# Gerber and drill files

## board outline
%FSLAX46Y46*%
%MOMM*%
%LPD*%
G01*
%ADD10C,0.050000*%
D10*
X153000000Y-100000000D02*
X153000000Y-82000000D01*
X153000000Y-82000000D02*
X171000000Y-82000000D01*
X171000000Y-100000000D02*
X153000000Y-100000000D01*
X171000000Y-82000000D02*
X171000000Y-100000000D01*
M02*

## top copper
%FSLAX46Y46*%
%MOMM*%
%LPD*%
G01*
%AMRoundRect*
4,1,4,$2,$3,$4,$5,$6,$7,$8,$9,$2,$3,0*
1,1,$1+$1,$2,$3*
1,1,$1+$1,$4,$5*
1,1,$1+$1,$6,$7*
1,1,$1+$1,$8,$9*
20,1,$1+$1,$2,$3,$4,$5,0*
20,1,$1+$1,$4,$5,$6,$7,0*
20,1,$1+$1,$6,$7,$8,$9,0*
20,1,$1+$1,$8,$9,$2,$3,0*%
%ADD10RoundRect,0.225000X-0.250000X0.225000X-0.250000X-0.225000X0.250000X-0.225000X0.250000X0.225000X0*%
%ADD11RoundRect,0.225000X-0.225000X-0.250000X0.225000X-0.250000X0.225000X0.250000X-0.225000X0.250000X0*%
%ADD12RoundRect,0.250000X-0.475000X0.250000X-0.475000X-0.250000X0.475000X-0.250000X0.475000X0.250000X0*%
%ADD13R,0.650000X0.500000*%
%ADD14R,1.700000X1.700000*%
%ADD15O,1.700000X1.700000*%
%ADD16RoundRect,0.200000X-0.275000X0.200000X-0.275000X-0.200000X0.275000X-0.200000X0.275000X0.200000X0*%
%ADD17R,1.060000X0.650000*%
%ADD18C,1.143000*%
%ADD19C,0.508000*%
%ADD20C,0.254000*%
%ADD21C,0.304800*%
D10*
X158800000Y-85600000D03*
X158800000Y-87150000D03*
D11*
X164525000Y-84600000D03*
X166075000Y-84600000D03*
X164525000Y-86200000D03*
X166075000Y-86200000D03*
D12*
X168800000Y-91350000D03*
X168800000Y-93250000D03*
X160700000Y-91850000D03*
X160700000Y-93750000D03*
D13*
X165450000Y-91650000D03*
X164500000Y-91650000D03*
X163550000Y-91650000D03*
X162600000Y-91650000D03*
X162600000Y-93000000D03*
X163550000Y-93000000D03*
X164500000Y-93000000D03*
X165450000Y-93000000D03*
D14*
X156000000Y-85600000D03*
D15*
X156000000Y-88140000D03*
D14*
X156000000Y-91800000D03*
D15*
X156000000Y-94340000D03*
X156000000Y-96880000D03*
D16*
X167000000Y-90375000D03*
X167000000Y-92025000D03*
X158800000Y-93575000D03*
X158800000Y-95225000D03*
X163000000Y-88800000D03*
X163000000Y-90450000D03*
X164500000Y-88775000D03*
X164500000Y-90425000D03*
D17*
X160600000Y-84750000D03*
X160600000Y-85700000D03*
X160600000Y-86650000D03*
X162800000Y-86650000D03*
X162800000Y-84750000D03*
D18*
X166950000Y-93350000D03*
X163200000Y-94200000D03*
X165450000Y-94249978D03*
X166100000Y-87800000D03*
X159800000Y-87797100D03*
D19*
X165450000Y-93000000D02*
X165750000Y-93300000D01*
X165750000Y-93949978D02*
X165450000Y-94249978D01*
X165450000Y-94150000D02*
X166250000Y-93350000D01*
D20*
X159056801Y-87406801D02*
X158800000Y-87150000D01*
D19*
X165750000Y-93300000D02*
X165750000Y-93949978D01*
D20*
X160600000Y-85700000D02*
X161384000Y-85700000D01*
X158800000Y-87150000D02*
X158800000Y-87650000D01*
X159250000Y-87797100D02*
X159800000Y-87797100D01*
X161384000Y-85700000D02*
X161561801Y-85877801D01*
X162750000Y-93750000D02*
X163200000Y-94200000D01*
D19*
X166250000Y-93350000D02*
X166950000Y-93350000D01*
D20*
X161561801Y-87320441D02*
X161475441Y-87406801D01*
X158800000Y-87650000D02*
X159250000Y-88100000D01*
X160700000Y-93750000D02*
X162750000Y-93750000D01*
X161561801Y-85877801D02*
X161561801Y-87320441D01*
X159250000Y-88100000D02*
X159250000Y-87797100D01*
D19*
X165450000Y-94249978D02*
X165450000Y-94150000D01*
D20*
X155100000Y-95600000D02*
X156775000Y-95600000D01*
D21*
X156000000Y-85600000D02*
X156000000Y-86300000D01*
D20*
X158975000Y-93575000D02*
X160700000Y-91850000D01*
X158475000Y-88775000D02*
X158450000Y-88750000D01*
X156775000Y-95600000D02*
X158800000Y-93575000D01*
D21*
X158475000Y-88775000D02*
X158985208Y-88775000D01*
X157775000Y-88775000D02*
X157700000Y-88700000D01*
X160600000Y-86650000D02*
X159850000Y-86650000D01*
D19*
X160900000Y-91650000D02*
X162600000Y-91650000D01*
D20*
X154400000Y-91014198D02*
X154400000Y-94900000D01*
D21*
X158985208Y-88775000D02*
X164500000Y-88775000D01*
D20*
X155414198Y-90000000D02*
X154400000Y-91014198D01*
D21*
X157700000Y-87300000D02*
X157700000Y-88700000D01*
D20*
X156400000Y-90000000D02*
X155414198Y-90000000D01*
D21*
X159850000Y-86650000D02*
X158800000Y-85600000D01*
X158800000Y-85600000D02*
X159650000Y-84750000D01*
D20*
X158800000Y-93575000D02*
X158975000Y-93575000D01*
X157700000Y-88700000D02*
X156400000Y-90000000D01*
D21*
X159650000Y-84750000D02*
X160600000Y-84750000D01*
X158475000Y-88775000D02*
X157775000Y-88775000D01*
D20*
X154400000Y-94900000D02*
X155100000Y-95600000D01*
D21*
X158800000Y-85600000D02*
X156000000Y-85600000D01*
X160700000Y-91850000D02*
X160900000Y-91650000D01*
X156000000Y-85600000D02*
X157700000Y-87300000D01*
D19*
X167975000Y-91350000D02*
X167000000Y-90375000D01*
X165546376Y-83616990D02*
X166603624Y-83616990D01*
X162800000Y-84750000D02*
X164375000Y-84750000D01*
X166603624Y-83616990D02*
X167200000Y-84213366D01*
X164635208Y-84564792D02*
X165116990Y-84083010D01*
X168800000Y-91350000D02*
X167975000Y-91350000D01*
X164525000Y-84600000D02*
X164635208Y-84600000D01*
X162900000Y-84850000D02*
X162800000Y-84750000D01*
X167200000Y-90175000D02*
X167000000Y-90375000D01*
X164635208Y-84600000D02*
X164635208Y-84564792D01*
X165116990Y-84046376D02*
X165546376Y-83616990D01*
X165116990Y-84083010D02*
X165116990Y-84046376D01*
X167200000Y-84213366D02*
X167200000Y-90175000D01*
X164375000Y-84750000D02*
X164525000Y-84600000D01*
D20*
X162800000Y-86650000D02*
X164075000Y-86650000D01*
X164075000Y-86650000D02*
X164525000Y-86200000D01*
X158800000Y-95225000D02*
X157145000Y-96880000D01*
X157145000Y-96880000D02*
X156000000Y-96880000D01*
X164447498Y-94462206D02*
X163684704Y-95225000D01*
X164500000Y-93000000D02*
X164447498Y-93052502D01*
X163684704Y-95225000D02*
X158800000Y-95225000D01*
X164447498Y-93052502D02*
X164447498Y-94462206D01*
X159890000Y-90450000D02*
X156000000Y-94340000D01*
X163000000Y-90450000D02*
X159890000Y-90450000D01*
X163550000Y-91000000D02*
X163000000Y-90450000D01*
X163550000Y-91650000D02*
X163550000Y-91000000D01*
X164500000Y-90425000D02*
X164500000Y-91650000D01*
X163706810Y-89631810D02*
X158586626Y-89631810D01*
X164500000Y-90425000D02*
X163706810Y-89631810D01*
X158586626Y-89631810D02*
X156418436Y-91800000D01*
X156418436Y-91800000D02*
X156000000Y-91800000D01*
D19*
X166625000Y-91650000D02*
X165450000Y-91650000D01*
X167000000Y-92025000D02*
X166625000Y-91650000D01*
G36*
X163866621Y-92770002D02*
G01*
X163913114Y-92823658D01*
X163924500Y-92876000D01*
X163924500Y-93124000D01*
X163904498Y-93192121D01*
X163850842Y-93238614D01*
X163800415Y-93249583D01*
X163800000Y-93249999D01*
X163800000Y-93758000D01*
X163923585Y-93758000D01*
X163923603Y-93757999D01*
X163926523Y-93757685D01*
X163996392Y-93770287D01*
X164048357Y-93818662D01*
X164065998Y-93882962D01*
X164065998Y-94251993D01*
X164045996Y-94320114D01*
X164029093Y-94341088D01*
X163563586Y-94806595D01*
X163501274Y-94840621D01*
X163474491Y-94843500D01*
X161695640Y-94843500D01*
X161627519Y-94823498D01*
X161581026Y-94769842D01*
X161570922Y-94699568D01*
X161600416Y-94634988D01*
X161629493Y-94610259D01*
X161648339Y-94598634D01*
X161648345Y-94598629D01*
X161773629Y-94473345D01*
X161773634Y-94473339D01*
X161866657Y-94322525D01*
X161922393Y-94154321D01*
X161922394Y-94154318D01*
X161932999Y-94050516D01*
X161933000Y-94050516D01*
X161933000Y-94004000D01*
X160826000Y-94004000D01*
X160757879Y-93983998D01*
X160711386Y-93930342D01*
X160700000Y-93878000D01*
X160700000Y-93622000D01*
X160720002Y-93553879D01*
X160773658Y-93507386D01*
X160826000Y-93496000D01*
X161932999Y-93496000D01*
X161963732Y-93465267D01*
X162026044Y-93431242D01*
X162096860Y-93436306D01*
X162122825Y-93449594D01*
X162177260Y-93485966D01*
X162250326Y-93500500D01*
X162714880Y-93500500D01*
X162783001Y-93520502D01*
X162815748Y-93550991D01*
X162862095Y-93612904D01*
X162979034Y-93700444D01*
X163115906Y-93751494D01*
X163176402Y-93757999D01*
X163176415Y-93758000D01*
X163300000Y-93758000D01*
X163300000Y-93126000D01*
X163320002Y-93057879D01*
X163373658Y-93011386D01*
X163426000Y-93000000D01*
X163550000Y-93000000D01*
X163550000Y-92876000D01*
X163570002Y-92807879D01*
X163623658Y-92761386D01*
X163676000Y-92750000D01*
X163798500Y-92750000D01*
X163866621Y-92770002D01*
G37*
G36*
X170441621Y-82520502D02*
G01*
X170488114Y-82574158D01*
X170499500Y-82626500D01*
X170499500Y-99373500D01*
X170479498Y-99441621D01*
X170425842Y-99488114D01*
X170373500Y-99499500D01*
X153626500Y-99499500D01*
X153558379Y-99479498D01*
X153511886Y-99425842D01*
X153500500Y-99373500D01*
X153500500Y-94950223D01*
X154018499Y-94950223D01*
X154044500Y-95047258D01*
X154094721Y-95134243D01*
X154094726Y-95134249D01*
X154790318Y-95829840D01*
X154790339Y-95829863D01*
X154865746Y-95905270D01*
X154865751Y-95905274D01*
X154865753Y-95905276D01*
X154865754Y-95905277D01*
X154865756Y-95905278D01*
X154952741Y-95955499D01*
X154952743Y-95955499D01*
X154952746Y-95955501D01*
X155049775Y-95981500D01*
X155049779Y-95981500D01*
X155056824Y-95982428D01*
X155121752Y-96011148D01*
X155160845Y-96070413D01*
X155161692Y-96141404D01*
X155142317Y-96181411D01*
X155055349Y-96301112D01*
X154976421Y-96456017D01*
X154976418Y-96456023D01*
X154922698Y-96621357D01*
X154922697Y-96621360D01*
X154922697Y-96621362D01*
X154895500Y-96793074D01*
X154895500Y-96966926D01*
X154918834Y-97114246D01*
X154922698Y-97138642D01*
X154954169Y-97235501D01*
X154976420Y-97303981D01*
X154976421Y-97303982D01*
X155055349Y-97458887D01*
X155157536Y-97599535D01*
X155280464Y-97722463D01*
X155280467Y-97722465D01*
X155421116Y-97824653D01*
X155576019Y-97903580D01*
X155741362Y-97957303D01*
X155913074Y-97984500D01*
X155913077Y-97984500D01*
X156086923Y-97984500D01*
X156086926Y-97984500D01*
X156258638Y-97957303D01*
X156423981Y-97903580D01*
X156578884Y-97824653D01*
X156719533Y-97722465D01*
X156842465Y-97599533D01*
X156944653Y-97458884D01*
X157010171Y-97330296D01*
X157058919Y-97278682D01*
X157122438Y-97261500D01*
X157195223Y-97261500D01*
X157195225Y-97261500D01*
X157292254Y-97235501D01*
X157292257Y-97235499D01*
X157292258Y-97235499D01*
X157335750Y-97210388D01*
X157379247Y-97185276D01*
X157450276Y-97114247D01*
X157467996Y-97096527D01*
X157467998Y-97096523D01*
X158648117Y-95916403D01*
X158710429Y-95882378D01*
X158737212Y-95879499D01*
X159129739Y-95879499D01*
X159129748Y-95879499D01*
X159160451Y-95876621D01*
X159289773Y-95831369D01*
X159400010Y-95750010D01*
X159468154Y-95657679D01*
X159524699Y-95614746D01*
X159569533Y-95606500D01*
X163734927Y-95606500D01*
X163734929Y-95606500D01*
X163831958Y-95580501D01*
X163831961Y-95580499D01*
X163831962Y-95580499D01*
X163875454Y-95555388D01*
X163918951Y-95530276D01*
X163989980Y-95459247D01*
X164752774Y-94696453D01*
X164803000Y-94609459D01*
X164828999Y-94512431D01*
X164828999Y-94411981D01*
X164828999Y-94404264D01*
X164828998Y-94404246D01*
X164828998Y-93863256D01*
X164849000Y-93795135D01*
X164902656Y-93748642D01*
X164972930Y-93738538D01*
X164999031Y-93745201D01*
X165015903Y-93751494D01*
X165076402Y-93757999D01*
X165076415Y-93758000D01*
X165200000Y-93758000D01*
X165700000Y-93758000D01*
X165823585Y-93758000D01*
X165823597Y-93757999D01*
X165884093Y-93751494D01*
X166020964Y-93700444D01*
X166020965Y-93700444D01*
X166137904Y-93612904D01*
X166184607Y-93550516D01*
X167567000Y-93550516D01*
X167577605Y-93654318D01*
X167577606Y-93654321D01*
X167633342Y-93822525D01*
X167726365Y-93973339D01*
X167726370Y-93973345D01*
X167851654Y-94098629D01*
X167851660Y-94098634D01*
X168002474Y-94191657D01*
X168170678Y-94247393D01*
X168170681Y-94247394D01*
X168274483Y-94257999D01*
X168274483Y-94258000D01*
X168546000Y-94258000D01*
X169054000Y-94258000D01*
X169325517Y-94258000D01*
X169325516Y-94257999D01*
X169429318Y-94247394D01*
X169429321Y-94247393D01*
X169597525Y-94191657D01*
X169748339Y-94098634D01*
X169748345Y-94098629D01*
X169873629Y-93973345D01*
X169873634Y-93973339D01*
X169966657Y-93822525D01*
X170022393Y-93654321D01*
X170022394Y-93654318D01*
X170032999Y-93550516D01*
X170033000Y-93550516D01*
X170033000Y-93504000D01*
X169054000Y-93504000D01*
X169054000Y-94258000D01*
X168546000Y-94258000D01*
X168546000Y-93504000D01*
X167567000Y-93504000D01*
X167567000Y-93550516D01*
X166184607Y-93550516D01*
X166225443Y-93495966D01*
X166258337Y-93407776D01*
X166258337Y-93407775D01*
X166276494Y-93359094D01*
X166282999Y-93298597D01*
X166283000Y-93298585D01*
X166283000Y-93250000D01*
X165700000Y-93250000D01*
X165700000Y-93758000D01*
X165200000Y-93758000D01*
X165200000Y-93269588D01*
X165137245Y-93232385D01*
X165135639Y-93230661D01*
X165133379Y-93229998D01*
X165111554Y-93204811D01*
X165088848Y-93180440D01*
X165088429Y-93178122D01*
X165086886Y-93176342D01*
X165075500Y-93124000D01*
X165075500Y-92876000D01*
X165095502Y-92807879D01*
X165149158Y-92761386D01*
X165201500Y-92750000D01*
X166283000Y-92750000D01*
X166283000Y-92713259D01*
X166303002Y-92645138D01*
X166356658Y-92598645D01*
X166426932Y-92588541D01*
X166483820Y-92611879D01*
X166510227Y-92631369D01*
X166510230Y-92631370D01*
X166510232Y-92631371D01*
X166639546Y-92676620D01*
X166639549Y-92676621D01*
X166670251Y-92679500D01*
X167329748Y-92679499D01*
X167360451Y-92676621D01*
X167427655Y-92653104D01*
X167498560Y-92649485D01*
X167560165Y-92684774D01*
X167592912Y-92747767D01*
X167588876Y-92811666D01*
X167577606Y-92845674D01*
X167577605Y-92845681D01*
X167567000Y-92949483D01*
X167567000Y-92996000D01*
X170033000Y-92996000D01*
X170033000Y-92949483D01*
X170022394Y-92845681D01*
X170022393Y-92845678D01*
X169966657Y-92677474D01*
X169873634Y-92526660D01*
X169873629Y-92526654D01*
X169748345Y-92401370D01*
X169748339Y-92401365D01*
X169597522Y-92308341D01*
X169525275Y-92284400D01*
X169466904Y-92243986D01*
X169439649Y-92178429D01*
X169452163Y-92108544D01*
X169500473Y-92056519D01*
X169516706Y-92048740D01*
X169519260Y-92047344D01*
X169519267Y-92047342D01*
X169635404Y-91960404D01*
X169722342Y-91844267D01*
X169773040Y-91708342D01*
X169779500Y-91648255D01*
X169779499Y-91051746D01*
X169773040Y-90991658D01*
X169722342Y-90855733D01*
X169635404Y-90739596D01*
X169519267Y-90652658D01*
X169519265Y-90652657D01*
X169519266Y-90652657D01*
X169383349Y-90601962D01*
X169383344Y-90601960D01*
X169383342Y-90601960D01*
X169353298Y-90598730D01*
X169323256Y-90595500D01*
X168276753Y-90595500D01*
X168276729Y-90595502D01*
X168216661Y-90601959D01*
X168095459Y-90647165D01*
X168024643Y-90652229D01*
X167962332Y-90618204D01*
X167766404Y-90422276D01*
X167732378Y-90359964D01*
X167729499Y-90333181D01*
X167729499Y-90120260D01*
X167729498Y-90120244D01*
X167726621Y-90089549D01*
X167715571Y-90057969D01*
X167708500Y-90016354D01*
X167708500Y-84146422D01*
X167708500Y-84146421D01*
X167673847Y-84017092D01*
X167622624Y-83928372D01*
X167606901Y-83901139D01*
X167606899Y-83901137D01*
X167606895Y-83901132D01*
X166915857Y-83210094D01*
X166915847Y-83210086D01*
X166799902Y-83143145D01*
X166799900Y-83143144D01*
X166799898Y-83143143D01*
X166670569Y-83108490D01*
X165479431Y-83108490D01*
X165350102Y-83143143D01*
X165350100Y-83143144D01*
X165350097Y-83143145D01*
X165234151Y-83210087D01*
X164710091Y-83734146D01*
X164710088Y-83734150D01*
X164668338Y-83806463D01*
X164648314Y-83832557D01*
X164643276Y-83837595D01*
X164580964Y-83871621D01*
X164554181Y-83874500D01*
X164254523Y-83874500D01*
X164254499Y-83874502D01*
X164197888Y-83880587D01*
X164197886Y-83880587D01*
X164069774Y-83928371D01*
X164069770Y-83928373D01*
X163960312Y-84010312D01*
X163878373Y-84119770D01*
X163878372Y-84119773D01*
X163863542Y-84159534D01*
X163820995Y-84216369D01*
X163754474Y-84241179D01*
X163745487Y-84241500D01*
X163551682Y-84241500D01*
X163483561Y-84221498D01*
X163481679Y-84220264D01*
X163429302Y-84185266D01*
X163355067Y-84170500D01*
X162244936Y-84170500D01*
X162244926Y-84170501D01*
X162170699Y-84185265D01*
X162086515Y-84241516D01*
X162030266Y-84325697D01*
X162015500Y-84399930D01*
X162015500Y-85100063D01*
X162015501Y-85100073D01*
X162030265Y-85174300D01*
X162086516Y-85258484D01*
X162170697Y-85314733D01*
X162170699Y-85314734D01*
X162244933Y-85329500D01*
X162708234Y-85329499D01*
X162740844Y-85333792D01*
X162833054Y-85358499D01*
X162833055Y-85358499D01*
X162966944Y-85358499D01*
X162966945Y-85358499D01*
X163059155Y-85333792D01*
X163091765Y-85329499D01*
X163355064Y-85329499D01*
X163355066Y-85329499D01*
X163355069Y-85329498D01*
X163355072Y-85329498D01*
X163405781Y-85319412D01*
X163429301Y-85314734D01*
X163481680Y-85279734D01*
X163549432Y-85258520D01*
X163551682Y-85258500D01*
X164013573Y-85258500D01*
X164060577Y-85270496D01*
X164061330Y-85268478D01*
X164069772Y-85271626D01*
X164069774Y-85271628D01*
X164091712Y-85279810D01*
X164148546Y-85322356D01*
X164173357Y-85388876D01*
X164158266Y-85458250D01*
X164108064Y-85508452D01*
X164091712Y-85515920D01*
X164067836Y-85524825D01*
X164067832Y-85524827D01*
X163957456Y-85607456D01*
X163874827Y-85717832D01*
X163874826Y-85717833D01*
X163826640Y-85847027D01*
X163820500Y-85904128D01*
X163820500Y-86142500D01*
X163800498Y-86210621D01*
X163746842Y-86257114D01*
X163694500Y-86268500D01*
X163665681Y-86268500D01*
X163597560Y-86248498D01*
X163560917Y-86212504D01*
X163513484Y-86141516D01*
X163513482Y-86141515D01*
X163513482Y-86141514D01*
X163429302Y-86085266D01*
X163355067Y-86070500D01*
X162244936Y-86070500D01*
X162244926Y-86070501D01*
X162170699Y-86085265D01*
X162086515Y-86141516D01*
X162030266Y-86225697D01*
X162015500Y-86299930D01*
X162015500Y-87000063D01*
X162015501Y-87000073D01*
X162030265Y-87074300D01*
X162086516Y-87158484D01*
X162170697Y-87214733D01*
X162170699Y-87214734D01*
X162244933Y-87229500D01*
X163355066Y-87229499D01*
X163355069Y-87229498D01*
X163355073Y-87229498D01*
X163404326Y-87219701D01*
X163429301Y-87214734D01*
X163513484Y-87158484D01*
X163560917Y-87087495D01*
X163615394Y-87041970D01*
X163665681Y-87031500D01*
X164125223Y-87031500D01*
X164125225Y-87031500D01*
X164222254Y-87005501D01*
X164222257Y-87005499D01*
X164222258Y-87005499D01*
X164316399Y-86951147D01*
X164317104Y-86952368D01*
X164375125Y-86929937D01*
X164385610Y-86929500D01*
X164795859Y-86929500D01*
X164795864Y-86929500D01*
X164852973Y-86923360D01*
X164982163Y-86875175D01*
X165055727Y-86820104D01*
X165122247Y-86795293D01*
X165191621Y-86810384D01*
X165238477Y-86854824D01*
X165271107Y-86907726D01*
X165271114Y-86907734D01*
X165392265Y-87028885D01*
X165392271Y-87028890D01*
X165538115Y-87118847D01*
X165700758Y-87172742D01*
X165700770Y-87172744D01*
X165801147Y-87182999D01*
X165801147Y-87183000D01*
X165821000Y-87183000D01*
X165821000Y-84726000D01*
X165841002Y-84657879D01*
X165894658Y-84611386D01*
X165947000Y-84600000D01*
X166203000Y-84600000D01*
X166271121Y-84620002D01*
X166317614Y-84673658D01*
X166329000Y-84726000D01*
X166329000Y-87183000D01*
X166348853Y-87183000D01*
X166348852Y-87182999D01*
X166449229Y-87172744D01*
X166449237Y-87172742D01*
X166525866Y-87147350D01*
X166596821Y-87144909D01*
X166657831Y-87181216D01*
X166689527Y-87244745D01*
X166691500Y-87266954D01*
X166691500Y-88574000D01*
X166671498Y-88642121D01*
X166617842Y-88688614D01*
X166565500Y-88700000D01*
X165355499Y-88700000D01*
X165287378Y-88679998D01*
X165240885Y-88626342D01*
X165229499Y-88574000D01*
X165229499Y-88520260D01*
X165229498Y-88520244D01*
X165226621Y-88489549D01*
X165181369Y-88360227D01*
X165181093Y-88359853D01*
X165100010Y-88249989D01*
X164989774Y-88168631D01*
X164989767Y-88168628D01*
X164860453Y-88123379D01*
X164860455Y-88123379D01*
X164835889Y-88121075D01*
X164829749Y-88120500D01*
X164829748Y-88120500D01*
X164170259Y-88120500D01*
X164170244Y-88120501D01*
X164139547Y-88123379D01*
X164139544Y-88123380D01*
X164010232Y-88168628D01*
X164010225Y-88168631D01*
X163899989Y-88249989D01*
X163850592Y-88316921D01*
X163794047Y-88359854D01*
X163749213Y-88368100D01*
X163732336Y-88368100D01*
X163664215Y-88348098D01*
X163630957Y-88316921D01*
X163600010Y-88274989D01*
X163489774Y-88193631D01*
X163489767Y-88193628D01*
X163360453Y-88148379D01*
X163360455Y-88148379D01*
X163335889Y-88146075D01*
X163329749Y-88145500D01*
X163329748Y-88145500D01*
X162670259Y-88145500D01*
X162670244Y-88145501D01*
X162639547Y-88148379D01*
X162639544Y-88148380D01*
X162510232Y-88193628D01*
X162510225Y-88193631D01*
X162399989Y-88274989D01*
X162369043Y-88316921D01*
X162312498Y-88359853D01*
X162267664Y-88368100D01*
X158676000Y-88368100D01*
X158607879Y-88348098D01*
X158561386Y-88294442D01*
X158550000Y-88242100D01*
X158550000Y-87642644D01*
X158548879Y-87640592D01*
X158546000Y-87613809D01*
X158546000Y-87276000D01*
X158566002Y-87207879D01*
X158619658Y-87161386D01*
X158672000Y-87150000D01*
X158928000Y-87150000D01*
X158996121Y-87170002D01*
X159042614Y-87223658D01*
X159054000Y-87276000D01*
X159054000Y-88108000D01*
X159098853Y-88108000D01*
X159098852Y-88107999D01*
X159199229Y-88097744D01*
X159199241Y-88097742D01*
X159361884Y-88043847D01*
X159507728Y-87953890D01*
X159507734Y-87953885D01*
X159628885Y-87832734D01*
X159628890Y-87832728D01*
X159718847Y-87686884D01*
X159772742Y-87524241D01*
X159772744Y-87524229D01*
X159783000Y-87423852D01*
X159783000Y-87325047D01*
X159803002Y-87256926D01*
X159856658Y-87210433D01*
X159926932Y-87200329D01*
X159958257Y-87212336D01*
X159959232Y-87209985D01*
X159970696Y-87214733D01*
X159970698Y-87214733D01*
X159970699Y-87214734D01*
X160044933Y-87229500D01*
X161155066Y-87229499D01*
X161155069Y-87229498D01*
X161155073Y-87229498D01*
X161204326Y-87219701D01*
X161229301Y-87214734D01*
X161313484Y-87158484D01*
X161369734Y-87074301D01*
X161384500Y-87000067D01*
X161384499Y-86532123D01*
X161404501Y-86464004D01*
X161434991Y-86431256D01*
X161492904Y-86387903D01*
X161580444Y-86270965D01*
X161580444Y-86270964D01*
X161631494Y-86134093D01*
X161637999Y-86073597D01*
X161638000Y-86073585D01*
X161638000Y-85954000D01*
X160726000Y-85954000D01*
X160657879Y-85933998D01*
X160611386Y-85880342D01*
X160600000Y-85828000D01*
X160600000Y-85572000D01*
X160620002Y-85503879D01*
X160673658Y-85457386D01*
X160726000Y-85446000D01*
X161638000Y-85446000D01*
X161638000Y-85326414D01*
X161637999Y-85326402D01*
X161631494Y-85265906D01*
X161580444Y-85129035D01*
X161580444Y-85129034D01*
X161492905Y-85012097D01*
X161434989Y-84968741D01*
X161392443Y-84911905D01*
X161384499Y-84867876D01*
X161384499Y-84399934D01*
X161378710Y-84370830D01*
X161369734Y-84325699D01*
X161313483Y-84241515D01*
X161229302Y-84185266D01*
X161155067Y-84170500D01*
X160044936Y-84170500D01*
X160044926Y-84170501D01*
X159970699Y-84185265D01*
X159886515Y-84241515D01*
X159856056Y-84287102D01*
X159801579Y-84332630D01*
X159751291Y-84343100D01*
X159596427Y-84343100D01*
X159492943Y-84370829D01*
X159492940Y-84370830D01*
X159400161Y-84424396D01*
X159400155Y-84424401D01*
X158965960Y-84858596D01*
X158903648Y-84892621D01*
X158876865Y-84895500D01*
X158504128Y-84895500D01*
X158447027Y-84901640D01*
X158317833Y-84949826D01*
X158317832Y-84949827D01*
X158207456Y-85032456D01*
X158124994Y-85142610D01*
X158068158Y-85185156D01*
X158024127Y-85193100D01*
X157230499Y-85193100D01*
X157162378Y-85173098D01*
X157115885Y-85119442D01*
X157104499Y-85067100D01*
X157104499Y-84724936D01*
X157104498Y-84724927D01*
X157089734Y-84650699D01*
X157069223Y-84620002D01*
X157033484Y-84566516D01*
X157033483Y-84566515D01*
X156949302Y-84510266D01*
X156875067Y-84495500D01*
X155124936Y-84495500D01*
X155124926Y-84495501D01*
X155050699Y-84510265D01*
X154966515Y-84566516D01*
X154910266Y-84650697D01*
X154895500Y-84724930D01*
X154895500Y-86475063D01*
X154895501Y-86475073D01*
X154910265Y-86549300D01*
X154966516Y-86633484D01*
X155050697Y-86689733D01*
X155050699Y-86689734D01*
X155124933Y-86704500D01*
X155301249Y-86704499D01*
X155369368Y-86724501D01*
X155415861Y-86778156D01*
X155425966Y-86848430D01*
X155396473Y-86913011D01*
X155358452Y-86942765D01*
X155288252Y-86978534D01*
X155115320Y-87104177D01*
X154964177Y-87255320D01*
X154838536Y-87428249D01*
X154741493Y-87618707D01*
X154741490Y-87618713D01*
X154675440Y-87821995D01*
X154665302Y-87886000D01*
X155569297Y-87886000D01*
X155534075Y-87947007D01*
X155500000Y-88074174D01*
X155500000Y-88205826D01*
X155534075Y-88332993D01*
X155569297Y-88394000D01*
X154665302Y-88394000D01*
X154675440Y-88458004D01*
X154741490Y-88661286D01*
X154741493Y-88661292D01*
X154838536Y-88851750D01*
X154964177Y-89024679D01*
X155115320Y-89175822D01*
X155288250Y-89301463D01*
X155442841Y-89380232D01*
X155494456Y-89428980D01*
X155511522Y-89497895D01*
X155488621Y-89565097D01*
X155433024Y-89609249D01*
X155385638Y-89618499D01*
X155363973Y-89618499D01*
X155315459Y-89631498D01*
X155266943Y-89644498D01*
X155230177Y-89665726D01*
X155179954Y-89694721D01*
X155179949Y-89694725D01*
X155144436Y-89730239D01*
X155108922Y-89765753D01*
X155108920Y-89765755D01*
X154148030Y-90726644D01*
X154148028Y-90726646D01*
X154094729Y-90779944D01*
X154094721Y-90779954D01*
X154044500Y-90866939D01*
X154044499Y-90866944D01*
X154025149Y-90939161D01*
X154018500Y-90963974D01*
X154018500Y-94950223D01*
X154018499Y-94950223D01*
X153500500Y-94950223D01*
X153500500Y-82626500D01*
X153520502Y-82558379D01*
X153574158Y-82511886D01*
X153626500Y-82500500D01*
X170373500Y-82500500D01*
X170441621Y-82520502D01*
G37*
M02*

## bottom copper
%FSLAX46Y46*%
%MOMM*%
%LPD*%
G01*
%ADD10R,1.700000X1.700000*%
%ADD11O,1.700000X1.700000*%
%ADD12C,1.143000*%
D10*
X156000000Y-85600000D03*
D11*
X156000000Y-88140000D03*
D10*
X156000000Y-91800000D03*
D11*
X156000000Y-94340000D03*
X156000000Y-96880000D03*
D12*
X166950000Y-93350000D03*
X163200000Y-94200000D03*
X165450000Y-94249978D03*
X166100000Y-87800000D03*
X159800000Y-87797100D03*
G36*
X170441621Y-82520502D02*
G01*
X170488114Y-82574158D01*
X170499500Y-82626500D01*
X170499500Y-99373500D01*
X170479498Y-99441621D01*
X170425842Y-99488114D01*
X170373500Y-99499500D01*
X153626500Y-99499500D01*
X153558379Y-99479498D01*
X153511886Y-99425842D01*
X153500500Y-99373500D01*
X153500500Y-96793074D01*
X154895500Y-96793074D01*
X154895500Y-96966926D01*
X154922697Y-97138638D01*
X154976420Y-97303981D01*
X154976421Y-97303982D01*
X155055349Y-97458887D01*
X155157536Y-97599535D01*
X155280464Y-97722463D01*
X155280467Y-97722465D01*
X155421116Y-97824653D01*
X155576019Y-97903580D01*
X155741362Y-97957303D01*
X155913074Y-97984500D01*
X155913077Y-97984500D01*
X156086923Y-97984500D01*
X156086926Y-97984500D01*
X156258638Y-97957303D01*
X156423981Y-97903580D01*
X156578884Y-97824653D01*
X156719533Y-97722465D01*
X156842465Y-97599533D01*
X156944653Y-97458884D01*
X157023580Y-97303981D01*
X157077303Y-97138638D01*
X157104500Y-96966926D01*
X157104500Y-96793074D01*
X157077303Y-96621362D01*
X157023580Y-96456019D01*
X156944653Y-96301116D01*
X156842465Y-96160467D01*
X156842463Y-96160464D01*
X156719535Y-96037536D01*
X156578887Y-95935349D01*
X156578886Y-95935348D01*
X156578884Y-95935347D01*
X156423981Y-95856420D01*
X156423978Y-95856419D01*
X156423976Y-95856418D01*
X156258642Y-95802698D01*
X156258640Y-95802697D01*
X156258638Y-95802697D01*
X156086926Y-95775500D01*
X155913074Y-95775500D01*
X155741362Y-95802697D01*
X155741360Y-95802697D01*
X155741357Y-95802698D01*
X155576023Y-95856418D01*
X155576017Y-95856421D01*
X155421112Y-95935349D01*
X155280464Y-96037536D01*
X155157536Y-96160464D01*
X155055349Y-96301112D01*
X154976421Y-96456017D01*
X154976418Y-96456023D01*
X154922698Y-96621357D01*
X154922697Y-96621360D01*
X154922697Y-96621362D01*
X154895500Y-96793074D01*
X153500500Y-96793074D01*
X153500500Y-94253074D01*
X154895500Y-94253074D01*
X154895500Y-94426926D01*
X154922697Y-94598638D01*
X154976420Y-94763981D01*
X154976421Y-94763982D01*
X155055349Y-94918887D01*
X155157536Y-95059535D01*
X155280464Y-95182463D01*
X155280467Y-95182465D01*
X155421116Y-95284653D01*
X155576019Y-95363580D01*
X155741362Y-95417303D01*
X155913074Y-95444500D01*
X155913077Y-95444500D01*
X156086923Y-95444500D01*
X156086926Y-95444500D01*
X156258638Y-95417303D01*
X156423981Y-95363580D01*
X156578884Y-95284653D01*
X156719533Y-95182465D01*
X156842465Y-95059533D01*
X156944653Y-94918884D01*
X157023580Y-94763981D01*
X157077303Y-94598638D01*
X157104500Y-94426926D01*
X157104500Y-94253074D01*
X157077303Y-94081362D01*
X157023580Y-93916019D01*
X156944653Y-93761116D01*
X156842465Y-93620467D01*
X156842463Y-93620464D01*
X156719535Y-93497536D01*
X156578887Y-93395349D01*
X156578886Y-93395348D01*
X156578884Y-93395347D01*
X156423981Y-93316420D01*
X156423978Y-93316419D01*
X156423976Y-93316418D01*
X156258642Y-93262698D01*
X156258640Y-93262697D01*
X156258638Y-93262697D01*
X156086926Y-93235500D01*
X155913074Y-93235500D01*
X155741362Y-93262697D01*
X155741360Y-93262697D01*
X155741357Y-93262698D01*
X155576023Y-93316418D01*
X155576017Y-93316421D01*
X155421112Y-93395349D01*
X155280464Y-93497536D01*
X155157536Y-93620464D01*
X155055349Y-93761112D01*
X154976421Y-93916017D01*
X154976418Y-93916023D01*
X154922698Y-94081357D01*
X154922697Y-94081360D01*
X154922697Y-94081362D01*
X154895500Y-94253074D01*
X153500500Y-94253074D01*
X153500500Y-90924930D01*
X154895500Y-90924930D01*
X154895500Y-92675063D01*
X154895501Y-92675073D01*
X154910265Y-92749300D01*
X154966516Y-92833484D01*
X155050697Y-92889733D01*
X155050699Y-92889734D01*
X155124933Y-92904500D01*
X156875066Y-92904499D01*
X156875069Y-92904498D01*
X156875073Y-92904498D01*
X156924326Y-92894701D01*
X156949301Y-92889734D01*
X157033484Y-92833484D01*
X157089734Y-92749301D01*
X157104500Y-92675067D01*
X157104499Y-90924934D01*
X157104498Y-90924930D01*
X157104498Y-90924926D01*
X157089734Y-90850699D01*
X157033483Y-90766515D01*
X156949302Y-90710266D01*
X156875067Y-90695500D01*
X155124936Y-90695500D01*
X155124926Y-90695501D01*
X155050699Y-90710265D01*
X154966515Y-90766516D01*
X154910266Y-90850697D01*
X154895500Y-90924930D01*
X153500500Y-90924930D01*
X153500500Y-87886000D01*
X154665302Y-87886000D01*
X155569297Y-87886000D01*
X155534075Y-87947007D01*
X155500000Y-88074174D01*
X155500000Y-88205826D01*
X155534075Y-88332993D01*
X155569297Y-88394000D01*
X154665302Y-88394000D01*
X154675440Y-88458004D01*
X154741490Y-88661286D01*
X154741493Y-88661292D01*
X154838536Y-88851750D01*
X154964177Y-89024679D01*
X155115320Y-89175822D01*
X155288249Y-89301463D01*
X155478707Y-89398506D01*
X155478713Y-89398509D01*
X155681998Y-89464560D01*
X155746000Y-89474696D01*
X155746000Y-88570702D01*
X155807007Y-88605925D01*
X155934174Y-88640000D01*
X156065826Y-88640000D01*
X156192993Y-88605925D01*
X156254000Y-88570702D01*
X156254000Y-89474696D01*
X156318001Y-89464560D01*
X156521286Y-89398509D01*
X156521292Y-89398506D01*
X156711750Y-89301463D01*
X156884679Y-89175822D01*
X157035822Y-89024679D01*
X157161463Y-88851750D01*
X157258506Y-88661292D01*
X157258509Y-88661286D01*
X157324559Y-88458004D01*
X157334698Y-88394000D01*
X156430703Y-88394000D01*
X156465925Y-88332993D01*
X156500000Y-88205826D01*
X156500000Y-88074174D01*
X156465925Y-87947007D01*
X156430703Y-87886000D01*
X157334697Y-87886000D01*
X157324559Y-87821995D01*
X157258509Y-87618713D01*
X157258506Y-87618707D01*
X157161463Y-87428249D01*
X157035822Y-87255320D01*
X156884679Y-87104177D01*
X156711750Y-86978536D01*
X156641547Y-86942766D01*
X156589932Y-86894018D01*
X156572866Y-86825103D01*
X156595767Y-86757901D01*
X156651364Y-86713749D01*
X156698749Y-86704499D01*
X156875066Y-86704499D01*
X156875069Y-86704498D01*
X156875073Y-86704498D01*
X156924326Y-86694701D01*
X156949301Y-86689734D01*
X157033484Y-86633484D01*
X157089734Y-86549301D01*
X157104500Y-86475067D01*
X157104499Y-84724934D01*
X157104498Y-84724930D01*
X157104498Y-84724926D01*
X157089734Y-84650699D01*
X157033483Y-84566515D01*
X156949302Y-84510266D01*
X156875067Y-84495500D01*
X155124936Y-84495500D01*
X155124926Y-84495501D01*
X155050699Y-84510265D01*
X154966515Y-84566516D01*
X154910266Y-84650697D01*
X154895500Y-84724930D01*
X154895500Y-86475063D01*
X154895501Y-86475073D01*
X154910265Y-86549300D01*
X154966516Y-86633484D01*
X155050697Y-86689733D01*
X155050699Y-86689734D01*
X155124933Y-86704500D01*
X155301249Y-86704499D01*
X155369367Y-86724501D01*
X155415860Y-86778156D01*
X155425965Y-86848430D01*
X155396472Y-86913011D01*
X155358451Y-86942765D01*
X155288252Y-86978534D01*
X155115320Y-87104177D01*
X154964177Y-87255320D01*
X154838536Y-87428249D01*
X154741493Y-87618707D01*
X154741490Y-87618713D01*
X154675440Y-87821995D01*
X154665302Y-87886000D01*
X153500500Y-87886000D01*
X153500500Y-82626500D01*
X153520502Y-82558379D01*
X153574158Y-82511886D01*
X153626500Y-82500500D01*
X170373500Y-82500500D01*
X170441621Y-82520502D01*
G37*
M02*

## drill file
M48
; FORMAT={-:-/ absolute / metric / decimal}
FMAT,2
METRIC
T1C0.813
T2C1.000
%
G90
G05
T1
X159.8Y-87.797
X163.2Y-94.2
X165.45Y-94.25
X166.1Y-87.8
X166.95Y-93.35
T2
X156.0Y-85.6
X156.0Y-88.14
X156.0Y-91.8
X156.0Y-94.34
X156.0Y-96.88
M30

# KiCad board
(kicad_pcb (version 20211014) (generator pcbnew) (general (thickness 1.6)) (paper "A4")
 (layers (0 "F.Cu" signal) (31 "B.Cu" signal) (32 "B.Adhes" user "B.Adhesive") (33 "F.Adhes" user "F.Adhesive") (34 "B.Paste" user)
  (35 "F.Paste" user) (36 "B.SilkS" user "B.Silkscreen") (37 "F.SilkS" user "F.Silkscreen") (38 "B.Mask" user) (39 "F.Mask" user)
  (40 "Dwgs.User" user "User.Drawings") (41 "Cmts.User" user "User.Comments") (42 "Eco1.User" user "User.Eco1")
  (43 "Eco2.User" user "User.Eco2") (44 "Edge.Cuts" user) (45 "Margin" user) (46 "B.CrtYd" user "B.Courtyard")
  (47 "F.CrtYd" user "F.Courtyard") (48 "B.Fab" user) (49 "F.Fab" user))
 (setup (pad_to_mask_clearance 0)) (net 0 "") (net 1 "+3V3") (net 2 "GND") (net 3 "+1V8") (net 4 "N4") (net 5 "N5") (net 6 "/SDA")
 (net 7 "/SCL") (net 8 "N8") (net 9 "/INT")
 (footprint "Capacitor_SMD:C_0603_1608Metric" (layer "F.Cu") (at 158.8 86.375 -90)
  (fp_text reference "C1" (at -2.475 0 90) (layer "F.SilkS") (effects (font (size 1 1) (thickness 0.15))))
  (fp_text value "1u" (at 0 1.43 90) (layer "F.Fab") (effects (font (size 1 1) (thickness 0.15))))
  (pad "1" smd roundrect locked (at -0.775 0 270) (size 0.9 0.95) (layers "F.Cu" "F.Paste" "F.Mask") (roundrect_rratio 0.25) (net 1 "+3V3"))
  (pad "2" smd roundrect locked (at 0.775 0 270) (size 0.9 0.95) (layers "F.Cu" "F.Paste" "F.Mask") (roundrect_rratio 0.25) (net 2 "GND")))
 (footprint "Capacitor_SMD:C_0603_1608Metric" (layer "F.Cu") (at 165.3 84.6) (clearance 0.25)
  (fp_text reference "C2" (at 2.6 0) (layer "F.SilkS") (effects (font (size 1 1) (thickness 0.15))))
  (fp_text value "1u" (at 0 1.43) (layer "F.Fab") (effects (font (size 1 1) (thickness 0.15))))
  (pad "1" smd roundrect locked (at -0.775 0) (size 0.9 0.95) (layers "F.Cu" "F.Paste" "F.Mask") (roundrect_rratio 0.25) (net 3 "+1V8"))
  (pad "2" smd roundrect locked (at 0.775 0) (size 0.9 0.95) (layers "F.Cu" "F.Paste" "F.Mask") (roundrect_rratio 0.25) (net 2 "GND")))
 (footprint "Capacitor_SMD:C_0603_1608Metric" (layer "F.Cu") (at 165.3 86.2)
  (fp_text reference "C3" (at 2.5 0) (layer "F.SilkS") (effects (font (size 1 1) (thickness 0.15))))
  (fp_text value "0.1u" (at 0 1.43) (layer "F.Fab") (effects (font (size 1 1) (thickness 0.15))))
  (pad "1" smd roundrect locked (at -0.775 0) (size 0.9 0.95) (layers "F.Cu" "F.Paste" "F.Mask") (roundrect_rratio 0.25) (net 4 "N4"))
  (pad "2" smd roundrect locked (at 0.775 0) (size 0.9 0.95) (layers "F.Cu" "F.Paste" "F.Mask") (roundrect_rratio 0.25) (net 2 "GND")))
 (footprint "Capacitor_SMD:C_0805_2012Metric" (layer "F.Cu") (at 168.8 92.3 -90)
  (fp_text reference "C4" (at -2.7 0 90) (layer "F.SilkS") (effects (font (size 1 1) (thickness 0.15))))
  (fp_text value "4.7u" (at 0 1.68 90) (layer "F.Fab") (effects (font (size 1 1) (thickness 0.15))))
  (pad "1" smd roundrect locked (at -0.95 0 270) (size 1 1.45) (layers "F.Cu" "F.Paste" "F.Mask") (roundrect_rratio 0.25) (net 3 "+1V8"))
  (pad "2" smd roundrect locked (at 0.95 0 270) (size 1 1.45) (layers "F.Cu" "F.Paste" "F.Mask") (roundrect_rratio 0.25) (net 2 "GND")))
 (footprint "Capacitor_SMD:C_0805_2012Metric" (layer "F.Cu") (at 160.7 92.8 -90)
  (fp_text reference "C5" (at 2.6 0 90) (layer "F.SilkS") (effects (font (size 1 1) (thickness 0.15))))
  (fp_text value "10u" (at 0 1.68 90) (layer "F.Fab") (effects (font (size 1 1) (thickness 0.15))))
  (pad "1" smd roundrect locked (at -0.95 0 270) (size 1 1.45) (layers "F.Cu" "F.Paste" "F.Mask") (roundrect_rratio 0.25) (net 1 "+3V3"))
  (pad "2" smd roundrect locked (at 0.95 0 270) (size 1 1.45) (layers "F.Cu" "F.Paste" "F.Mask") (roundrect_rratio 0.25) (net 2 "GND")))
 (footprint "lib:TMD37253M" (layer "F.Cu") (at 164.025 92.325 -90) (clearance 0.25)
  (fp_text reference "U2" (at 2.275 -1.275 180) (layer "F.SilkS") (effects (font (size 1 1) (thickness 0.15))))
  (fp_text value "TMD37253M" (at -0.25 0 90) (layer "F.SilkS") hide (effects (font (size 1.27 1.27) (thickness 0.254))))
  (pad "1" smd rect locked (at -0.675 -1.425 270) (size 0.5 0.65) (layers "F.Cu" "F.Paste" "F.Mask") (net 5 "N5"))
  (pad "2" smd rect locked (at -0.675 -0.475 270) (size 0.5 0.65) (layers "F.Cu" "F.Paste" "F.Mask") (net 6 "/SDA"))
  (pad "3" smd rect locked (at -0.675 0.475 270) (size 0.5 0.65) (layers "F.Cu" "F.Paste" "F.Mask") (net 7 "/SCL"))
  (pad "4" smd rect locked (at -0.675 1.425 270) (size 0.5 0.65) (layers "F.Cu" "F.Paste" "F.Mask") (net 1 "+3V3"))
  (pad "5" smd rect locked (at 0.675 1.425 270) (size 0.5 0.65) (layers "F.Cu" "F.Paste" "F.Mask") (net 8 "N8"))
  (pad "6" smd rect locked (at 0.675 0.475 270) (size 0.5 0.65) (layers "F.Cu" "F.Paste" "F.Mask") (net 2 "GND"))
  (pad "7" smd rect locked (at 0.675 -0.475 270) (size 0.5 0.65) (layers "F.Cu" "F.Paste" "F.Mask") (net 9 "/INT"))
  (pad "8" smd rect locked (at 0.675 -1.425 270) (size 0.5 0.65) (layers "F.Cu" "F.Paste" "F.Mask") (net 2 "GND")))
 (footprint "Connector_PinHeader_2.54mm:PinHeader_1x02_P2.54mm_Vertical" (layer "F.Cu") (at 156 85.6)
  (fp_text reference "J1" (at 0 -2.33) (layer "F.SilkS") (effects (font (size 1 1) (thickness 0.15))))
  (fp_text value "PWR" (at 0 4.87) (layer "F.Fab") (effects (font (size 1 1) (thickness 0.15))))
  (pad "1" thru_hole rect locked (at 0 0) (size 1.7 1.7) (drill 1) (layers *.Cu *.Mask) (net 1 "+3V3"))
  (pad "2" thru_hole oval locked (at 0 2.54) (size 1.7 1.7) (drill 1) (layers *.Cu *.Mask) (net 2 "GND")))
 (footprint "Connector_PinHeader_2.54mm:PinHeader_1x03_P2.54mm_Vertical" (layer "F.Cu") (at 156 91.8)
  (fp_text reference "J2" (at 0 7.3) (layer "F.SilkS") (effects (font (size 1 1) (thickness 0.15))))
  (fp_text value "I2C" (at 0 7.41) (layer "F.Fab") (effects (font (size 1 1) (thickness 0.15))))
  (pad "1" thru_hole rect locked (at 0 0) (size 1.7 1.7) (drill 1) (layers *.Cu *.Mask) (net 6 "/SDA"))
  (pad "2" thru_hole oval locked (at 0 2.54) (size 1.7 1.7) (drill 1) (layers *.Cu *.Mask) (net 7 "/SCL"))
  (pad "3" thru_hole oval locked (at 0 5.08) (size 1.7 1.7) (drill 1) (layers *.Cu *.Mask) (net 9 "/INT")))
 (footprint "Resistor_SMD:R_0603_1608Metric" (layer "F.Cu") (at 167 91.2 -90)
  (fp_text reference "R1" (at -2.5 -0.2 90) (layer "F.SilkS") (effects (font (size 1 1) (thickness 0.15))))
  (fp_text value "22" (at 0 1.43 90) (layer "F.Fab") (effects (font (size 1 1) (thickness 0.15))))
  (pad "1" smd roundrect locked (at -0.825 0 270) (size 0.8 0.95) (layers "F.Cu" "F.Paste" "F.Mask") (roundrect_rratio 0.25) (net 3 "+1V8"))
  (pad "2" smd roundrect locked (at 0.825 0 270) (size 0.8 0.95) (layers "F.Cu" "F.Paste" "F.Mask") (roundrect_rratio 0.25) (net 5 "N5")))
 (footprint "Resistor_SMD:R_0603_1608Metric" (layer "F.Cu") (at 158.8 94.4 -90)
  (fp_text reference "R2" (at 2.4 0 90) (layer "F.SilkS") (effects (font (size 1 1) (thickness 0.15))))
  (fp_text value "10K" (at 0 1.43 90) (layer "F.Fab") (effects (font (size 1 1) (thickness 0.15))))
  (pad "1" smd roundrect locked (at -0.825 0 270) (size 0.8 0.95) (layers "F.Cu" "F.Paste" "F.Mask") (roundrect_rratio 0.25) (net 1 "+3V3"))
  (pad "2" smd roundrect locked (at 0.825 0 270) (size 0.8 0.95) (layers "F.Cu" "F.Paste" "F.Mask") (roundrect_rratio 0.25) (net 9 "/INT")))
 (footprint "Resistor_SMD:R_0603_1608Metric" (layer "F.Cu") (at 163 89.625 -90)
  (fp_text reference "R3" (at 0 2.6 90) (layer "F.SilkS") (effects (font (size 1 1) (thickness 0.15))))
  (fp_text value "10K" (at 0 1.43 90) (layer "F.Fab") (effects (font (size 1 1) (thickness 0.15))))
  (pad "1" smd roundrect locked (at -0.825 0 270) (size 0.8 0.95) (layers "F.Cu" "F.Paste" "F.Mask") (roundrect_rratio 0.25) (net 1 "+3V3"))
  (pad "2" smd roundrect locked (at 0.825 0 270) (size 0.8 0.95) (layers "F.Cu" "F.Paste" "F.Mask") (roundrect_rratio 0.25) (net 7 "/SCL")))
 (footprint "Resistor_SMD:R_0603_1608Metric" (layer "F.Cu") (at 164.5 89.6 -90)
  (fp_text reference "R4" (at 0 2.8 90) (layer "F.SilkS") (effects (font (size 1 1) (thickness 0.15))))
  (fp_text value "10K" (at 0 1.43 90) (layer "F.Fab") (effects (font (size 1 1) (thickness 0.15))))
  (pad "1" smd roundrect locked (at -0.825 0 270) (size 0.8 0.95) (layers "F.Cu" "F.Paste" "F.Mask") (roundrect_rratio 0.25) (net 1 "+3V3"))
  (pad "2" smd roundrect locked (at 0.825 0 270) (size 0.8 0.95) (layers "F.Cu" "F.Paste" "F.Mask") (roundrect_rratio 0.25) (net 6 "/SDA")))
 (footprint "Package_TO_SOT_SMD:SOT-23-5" (layer "F.Cu") (at 161.7 85.7)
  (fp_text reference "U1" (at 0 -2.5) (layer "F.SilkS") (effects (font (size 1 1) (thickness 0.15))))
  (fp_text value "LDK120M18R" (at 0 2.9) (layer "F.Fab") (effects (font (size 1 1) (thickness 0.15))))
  (pad "1" smd rect locked (at -1.1 -0.95) (size 1.06 0.65) (layers "F.Cu" "F.Paste" "F.Mask") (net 1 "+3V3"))
  (pad "2" smd rect locked (at -1.1 0) (size 1.06 0.65) (layers "F.Cu" "F.Paste" "F.Mask") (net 2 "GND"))
  (pad "3" smd rect locked (at -1.1 0.95) (size 1.06 0.65) (layers "F.Cu" "F.Paste" "F.Mask") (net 1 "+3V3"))
  (pad "4" smd rect locked (at 1.1 0.95) (size 1.06 0.65) (layers "F.Cu" "F.Paste" "F.Mask") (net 4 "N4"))
  (pad "5" smd rect locked (at 1.1 -0.95) (size 1.06 0.65) (layers "F.Cu" "F.Paste" "F.Mask") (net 3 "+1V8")))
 (gr_line (start 153 100) (end 153 82) (layer "Edge.Cuts") (width 0.05))
 (gr_line (start 153 82) (end 171 82) (layer "Edge.Cuts") (width 0.05))
 (gr_line (start 171 100) (end 153 100) (layer "Edge.Cuts") (width 0.05))
 (gr_line (start 171 82) (end 171 100) (layer "Edge.Cuts") (width 0.05))
 (segment (start 165.45 93) (end 165.75 93.3) (width 0.508) (layer "F.Cu") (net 2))
 (segment (start 165.75 93.949978) (end 165.45 94.249978) (width 0.508) (layer "F.Cu") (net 2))
 (segment (start 165.45 94.15) (end 166.25 93.35) (width 0.508) (layer "F.Cu") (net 2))
 (segment (start 159.056801 87.406801) (end 158.8 87.15) (width 0.254) (layer "F.Cu") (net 2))
 (segment (start 165.75 93.3) (end 165.75 93.949978) (width 0.508) (layer "F.Cu") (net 2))
 (segment (start 160.6 85.7) (end 161.384 85.7) (width 0.254) (layer "F.Cu") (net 2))
 (segment (start 158.8 87.15) (end 158.8 87.65) (width 0.254) (layer "F.Cu") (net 2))
 (segment (start 159.25 87.7971) (end 159.8 87.7971) (width 0.254) (layer "F.Cu") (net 2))
 (segment (start 161.384 85.7) (end 161.561801 85.877801) (width 0.254) (layer "F.Cu") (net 2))
 (segment (start 162.75 93.75) (end 163.2 94.2) (width 0.254) (layer "F.Cu") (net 2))
 (segment (start 166.25 93.35) (end 166.95 93.35) (width 0.508) (layer "F.Cu") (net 2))
 (segment (start 161.561801 87.320441) (end 161.475441 87.406801) (width 0.254) (layer "F.Cu") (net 2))
 (segment (start 158.8 87.65) (end 159.25 88.1) (width 0.254) (layer "F.Cu") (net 2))
 (segment (start 160.7 93.75) (end 162.75 93.75) (width 0.254) (layer "F.Cu") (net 2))
 (segment (start 161.561801 85.877801) (end 161.561801 87.320441) (width 0.254) (layer "F.Cu") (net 2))
 (segment (start 159.25 88.1) (end 159.25 87.7971) (width 0.254) (layer "F.Cu") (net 2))
 (segment (start 165.45 94.249978) (end 165.45 94.15) (width 0.508) (layer "F.Cu") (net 2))
 (via (at 166.95 93.35) (size 1.143) (drill 0.8128) (layers "F.Cu" "B.Cu") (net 2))
 (via (at 163.2 94.2) (size 1.143) (drill 0.8128) (layers "F.Cu" "B.Cu") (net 2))
 (via (at 165.45 94.249978) (size 1.143) (drill 0.8128) (layers "F.Cu" "B.Cu") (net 2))
 (via (at 166.1 87.8) (size 1.143) (drill 0.8128) (layers "F.Cu" "B.Cu") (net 2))
 (via (at 159.8 87.7971) (size 1.143) (drill 0.8128) (layers "F.Cu" "B.Cu") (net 2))
 (segment (start 155.1 95.6) (end 156.775 95.6) (width 0.254) (layer "F.Cu") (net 1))
 (segment (start 156 85.6) (end 156 86.3) (width 0.3048) (layer "F.Cu") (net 1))
 (segment (start 158.975 93.575) (end 160.7 91.85) (width 0.254) (layer "F.Cu") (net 1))
 (segment (start 158.475 88.775) (end 158.45 88.75) (width 0.254) (layer "F.Cu") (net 1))
 (segment (start 156.775 95.6) (end 158.8 93.575) (width 0.254) (layer "F.Cu") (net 1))
 (segment (start 158.475 88.775) (end 158.985208 88.775) (width 0.3048) (layer "F.Cu") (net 1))
 (segment (start 157.775 88.775) (end 157.7 88.7) (width 0.3048) (layer "F.Cu") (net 1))
 (segment (start 160.6 86.65) (end 159.85 86.65) (width 0.3048) (layer "F.Cu") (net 1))
 (segment (start 160.9 91.65) (end 162.6 91.65) (width 0.508) (layer "F.Cu") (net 1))
 (segment (start 154.4 91.014198) (end 154.4 94.9) (width 0.254) (layer "F.Cu") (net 1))
 (segment (start 158.985208 88.775) (end 164.5 88.775) (width 0.3048) (layer "F.Cu") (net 1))
 (segment (start 155.414198 90) (end 154.4 91.014198) (width 0.254) (layer "F.Cu") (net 1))
 (segment (start 157.7 87.3) (end 157.7 88.7) (width 0.3048) (layer "F.Cu") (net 1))
 (segment (start 156.4 90) (end 155.414198 90) (width 0.254) (layer "F.Cu") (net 1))
 (segment (start 159.85 86.65) (end 158.8 85.6) (width 0.3048) (layer "F.Cu") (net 1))
 (segment (start 158.8 85.6) (end 159.65 84.75) (width 0.3048) (layer "F.Cu") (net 1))
 (segment (start 158.8 93.575) (end 158.975 93.575) (width 0.254) (layer "F.Cu") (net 1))
 (segment (start 157.7 88.7) (end 156.4 90) (width 0.254) (layer "F.Cu") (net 1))
 (segment (start 159.65 84.75) (end 160.6 84.75) (width 0.3048) (layer "F.Cu") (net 1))
 (segment (start 158.475 88.775) (end 157.775 88.775) (width 0.3048) (layer "F.Cu") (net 1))
 (segment (start 154.4 94.9) (end 155.1 95.6) (width 0.254) (layer "F.Cu") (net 1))
 (segment (start 158.8 85.6) (end 156 85.6) (width 0.3048) (layer "F.Cu") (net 1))
 (segment (start 160.7 91.85) (end 160.9 91.65) (width 0.3048) (layer "F.Cu") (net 1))
 (segment (start 156 85.6) (end 157.7 87.3) (width 0.3048) (layer "F.Cu") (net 1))
 (segment (start 167.975 91.35) (end 167 90.375) (width 0.508) (layer "F.Cu") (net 3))
 (segment (start 165.546376 83.61699) (end 166.603624 83.61699) (width 0.508) (layer "F.Cu") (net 3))
 (segment (start 162.8 84.75) (end 164.375 84.75) (width 0.508) (layer "F.Cu") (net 3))
 (segment (start 166.603624 83.61699) (end 167.2 84.213366) (width 0.508) (layer "F.Cu") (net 3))
 (segment (start 164.635208 84.564792) (end 165.11699 84.08301) (width 0.508) (layer "F.Cu") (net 3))
 (segment (start 168.8 91.35) (end 167.975 91.35) (width 0.508) (layer "F.Cu") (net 3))
 (segment (start 164.525 84.6) (end 164.635208 84.6) (width 0.508) (layer "F.Cu") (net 3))
 (segment (start 162.9 84.85) (end 162.8 84.75) (width 0.508) (layer "F.Cu") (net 3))
 (segment (start 167.2 90.175) (end 167 90.375) (width 0.508) (layer "F.Cu") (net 3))
 (segment (start 164.635208 84.6) (end 164.635208 84.564792) (width 0.508) (layer "F.Cu") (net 3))
 (segment (start 165.11699 84.046376) (end 165.546376 83.61699) (width 0.508) (layer "F.Cu") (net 3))
 (segment (start 165.11699 84.08301) (end 165.11699 84.046376) (width 0.508) (layer "F.Cu") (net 3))
 (segment (start 167.2 84.213366) (end 167.2 90.175) (width 0.508) (layer "F.Cu") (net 3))
 (segment (start 164.375 84.75) (end 164.525 84.6) (width 0.508) (layer "F.Cu") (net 3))
 (segment (start 162.8 86.65) (end 164.075 86.65) (width 0.254) (layer "F.Cu") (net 4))
 (segment (start 164.075 86.65) (end 164.525 86.2) (width 0.254) (layer "F.Cu") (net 4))
 (segment (start 158.8 95.225) (end 157.145 96.88) (width 0.254) (layer "F.Cu") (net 9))
 (segment (start 157.145 96.88) (end 156 96.88) (width 0.254) (layer "F.Cu") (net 9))
 (segment (start 164.447498 94.462206) (end 163.684704 95.225) (width 0.254) (layer "F.Cu") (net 9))
 (segment (start 164.5 93) (end 164.447498 93.052502) (width 0.254) (layer "F.Cu") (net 9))
 (segment (start 163.684704 95.225) (end 158.8 95.225) (width 0.254) (layer "F.Cu") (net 9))
 (segment (start 164.447498 93.052502) (end 164.447498 94.462206) (width 0.254) (layer "F.Cu") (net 9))
 (segment (start 159.89 90.45) (end 156 94.34) (width 0.254) (layer "F.Cu") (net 7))
 (segment (start 163 90.45) (end 159.89 90.45) (width 0.254) (layer "F.Cu") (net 7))
 (segment (start 163.55 91) (end 163 90.45) (width 0.254) (layer "F.Cu") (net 7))
 (segment (start 163.55 91.65) (end 163.55 91) (width 0.254) (layer "F.Cu") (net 7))
 (segment (start 164.5 90.425) (end 164.5 91.65) (width 0.254) (layer "F.Cu") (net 6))
 (segment (start 163.70681 89.63181) (end 158.586626 89.63181) (width 0.254) (layer "F.Cu") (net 6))
 (segment (start 164.5 90.425) (end 163.70681 89.63181) (width 0.254) (layer "F.Cu") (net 6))
 (segment (start 158.586626 89.63181) (end 156.418436 91.8) (width 0.254) (layer "F.Cu") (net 6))
 (segment (start 156.418436 91.8) (end 156 91.8) (width 0.254) (layer "F.Cu") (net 6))
 (segment (start 166.625 91.65) (end 165.45 91.65) (width 0.508) (layer "F.Cu") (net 5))
 (segment (start 167 92.025) (end 166.625 91.65) (width 0.508) (layer "F.Cu") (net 5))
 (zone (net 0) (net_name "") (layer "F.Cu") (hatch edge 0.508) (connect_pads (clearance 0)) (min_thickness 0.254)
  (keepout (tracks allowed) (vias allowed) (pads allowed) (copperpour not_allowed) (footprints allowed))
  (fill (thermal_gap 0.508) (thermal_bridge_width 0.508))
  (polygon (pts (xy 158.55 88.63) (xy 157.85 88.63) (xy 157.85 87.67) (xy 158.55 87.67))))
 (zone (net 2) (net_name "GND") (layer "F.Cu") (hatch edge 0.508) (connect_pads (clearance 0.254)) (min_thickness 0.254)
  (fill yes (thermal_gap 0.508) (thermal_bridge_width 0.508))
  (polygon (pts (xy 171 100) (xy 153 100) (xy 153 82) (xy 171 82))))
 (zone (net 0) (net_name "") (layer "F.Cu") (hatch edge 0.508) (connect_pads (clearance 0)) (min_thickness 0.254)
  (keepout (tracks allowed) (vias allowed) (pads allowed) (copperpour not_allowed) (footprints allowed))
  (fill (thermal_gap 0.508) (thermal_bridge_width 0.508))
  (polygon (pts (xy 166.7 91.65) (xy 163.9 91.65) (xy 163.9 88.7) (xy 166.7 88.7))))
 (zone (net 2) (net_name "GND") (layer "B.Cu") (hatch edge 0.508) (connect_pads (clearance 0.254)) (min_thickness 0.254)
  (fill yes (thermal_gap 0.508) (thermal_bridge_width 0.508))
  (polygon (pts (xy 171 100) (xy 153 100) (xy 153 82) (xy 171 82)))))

